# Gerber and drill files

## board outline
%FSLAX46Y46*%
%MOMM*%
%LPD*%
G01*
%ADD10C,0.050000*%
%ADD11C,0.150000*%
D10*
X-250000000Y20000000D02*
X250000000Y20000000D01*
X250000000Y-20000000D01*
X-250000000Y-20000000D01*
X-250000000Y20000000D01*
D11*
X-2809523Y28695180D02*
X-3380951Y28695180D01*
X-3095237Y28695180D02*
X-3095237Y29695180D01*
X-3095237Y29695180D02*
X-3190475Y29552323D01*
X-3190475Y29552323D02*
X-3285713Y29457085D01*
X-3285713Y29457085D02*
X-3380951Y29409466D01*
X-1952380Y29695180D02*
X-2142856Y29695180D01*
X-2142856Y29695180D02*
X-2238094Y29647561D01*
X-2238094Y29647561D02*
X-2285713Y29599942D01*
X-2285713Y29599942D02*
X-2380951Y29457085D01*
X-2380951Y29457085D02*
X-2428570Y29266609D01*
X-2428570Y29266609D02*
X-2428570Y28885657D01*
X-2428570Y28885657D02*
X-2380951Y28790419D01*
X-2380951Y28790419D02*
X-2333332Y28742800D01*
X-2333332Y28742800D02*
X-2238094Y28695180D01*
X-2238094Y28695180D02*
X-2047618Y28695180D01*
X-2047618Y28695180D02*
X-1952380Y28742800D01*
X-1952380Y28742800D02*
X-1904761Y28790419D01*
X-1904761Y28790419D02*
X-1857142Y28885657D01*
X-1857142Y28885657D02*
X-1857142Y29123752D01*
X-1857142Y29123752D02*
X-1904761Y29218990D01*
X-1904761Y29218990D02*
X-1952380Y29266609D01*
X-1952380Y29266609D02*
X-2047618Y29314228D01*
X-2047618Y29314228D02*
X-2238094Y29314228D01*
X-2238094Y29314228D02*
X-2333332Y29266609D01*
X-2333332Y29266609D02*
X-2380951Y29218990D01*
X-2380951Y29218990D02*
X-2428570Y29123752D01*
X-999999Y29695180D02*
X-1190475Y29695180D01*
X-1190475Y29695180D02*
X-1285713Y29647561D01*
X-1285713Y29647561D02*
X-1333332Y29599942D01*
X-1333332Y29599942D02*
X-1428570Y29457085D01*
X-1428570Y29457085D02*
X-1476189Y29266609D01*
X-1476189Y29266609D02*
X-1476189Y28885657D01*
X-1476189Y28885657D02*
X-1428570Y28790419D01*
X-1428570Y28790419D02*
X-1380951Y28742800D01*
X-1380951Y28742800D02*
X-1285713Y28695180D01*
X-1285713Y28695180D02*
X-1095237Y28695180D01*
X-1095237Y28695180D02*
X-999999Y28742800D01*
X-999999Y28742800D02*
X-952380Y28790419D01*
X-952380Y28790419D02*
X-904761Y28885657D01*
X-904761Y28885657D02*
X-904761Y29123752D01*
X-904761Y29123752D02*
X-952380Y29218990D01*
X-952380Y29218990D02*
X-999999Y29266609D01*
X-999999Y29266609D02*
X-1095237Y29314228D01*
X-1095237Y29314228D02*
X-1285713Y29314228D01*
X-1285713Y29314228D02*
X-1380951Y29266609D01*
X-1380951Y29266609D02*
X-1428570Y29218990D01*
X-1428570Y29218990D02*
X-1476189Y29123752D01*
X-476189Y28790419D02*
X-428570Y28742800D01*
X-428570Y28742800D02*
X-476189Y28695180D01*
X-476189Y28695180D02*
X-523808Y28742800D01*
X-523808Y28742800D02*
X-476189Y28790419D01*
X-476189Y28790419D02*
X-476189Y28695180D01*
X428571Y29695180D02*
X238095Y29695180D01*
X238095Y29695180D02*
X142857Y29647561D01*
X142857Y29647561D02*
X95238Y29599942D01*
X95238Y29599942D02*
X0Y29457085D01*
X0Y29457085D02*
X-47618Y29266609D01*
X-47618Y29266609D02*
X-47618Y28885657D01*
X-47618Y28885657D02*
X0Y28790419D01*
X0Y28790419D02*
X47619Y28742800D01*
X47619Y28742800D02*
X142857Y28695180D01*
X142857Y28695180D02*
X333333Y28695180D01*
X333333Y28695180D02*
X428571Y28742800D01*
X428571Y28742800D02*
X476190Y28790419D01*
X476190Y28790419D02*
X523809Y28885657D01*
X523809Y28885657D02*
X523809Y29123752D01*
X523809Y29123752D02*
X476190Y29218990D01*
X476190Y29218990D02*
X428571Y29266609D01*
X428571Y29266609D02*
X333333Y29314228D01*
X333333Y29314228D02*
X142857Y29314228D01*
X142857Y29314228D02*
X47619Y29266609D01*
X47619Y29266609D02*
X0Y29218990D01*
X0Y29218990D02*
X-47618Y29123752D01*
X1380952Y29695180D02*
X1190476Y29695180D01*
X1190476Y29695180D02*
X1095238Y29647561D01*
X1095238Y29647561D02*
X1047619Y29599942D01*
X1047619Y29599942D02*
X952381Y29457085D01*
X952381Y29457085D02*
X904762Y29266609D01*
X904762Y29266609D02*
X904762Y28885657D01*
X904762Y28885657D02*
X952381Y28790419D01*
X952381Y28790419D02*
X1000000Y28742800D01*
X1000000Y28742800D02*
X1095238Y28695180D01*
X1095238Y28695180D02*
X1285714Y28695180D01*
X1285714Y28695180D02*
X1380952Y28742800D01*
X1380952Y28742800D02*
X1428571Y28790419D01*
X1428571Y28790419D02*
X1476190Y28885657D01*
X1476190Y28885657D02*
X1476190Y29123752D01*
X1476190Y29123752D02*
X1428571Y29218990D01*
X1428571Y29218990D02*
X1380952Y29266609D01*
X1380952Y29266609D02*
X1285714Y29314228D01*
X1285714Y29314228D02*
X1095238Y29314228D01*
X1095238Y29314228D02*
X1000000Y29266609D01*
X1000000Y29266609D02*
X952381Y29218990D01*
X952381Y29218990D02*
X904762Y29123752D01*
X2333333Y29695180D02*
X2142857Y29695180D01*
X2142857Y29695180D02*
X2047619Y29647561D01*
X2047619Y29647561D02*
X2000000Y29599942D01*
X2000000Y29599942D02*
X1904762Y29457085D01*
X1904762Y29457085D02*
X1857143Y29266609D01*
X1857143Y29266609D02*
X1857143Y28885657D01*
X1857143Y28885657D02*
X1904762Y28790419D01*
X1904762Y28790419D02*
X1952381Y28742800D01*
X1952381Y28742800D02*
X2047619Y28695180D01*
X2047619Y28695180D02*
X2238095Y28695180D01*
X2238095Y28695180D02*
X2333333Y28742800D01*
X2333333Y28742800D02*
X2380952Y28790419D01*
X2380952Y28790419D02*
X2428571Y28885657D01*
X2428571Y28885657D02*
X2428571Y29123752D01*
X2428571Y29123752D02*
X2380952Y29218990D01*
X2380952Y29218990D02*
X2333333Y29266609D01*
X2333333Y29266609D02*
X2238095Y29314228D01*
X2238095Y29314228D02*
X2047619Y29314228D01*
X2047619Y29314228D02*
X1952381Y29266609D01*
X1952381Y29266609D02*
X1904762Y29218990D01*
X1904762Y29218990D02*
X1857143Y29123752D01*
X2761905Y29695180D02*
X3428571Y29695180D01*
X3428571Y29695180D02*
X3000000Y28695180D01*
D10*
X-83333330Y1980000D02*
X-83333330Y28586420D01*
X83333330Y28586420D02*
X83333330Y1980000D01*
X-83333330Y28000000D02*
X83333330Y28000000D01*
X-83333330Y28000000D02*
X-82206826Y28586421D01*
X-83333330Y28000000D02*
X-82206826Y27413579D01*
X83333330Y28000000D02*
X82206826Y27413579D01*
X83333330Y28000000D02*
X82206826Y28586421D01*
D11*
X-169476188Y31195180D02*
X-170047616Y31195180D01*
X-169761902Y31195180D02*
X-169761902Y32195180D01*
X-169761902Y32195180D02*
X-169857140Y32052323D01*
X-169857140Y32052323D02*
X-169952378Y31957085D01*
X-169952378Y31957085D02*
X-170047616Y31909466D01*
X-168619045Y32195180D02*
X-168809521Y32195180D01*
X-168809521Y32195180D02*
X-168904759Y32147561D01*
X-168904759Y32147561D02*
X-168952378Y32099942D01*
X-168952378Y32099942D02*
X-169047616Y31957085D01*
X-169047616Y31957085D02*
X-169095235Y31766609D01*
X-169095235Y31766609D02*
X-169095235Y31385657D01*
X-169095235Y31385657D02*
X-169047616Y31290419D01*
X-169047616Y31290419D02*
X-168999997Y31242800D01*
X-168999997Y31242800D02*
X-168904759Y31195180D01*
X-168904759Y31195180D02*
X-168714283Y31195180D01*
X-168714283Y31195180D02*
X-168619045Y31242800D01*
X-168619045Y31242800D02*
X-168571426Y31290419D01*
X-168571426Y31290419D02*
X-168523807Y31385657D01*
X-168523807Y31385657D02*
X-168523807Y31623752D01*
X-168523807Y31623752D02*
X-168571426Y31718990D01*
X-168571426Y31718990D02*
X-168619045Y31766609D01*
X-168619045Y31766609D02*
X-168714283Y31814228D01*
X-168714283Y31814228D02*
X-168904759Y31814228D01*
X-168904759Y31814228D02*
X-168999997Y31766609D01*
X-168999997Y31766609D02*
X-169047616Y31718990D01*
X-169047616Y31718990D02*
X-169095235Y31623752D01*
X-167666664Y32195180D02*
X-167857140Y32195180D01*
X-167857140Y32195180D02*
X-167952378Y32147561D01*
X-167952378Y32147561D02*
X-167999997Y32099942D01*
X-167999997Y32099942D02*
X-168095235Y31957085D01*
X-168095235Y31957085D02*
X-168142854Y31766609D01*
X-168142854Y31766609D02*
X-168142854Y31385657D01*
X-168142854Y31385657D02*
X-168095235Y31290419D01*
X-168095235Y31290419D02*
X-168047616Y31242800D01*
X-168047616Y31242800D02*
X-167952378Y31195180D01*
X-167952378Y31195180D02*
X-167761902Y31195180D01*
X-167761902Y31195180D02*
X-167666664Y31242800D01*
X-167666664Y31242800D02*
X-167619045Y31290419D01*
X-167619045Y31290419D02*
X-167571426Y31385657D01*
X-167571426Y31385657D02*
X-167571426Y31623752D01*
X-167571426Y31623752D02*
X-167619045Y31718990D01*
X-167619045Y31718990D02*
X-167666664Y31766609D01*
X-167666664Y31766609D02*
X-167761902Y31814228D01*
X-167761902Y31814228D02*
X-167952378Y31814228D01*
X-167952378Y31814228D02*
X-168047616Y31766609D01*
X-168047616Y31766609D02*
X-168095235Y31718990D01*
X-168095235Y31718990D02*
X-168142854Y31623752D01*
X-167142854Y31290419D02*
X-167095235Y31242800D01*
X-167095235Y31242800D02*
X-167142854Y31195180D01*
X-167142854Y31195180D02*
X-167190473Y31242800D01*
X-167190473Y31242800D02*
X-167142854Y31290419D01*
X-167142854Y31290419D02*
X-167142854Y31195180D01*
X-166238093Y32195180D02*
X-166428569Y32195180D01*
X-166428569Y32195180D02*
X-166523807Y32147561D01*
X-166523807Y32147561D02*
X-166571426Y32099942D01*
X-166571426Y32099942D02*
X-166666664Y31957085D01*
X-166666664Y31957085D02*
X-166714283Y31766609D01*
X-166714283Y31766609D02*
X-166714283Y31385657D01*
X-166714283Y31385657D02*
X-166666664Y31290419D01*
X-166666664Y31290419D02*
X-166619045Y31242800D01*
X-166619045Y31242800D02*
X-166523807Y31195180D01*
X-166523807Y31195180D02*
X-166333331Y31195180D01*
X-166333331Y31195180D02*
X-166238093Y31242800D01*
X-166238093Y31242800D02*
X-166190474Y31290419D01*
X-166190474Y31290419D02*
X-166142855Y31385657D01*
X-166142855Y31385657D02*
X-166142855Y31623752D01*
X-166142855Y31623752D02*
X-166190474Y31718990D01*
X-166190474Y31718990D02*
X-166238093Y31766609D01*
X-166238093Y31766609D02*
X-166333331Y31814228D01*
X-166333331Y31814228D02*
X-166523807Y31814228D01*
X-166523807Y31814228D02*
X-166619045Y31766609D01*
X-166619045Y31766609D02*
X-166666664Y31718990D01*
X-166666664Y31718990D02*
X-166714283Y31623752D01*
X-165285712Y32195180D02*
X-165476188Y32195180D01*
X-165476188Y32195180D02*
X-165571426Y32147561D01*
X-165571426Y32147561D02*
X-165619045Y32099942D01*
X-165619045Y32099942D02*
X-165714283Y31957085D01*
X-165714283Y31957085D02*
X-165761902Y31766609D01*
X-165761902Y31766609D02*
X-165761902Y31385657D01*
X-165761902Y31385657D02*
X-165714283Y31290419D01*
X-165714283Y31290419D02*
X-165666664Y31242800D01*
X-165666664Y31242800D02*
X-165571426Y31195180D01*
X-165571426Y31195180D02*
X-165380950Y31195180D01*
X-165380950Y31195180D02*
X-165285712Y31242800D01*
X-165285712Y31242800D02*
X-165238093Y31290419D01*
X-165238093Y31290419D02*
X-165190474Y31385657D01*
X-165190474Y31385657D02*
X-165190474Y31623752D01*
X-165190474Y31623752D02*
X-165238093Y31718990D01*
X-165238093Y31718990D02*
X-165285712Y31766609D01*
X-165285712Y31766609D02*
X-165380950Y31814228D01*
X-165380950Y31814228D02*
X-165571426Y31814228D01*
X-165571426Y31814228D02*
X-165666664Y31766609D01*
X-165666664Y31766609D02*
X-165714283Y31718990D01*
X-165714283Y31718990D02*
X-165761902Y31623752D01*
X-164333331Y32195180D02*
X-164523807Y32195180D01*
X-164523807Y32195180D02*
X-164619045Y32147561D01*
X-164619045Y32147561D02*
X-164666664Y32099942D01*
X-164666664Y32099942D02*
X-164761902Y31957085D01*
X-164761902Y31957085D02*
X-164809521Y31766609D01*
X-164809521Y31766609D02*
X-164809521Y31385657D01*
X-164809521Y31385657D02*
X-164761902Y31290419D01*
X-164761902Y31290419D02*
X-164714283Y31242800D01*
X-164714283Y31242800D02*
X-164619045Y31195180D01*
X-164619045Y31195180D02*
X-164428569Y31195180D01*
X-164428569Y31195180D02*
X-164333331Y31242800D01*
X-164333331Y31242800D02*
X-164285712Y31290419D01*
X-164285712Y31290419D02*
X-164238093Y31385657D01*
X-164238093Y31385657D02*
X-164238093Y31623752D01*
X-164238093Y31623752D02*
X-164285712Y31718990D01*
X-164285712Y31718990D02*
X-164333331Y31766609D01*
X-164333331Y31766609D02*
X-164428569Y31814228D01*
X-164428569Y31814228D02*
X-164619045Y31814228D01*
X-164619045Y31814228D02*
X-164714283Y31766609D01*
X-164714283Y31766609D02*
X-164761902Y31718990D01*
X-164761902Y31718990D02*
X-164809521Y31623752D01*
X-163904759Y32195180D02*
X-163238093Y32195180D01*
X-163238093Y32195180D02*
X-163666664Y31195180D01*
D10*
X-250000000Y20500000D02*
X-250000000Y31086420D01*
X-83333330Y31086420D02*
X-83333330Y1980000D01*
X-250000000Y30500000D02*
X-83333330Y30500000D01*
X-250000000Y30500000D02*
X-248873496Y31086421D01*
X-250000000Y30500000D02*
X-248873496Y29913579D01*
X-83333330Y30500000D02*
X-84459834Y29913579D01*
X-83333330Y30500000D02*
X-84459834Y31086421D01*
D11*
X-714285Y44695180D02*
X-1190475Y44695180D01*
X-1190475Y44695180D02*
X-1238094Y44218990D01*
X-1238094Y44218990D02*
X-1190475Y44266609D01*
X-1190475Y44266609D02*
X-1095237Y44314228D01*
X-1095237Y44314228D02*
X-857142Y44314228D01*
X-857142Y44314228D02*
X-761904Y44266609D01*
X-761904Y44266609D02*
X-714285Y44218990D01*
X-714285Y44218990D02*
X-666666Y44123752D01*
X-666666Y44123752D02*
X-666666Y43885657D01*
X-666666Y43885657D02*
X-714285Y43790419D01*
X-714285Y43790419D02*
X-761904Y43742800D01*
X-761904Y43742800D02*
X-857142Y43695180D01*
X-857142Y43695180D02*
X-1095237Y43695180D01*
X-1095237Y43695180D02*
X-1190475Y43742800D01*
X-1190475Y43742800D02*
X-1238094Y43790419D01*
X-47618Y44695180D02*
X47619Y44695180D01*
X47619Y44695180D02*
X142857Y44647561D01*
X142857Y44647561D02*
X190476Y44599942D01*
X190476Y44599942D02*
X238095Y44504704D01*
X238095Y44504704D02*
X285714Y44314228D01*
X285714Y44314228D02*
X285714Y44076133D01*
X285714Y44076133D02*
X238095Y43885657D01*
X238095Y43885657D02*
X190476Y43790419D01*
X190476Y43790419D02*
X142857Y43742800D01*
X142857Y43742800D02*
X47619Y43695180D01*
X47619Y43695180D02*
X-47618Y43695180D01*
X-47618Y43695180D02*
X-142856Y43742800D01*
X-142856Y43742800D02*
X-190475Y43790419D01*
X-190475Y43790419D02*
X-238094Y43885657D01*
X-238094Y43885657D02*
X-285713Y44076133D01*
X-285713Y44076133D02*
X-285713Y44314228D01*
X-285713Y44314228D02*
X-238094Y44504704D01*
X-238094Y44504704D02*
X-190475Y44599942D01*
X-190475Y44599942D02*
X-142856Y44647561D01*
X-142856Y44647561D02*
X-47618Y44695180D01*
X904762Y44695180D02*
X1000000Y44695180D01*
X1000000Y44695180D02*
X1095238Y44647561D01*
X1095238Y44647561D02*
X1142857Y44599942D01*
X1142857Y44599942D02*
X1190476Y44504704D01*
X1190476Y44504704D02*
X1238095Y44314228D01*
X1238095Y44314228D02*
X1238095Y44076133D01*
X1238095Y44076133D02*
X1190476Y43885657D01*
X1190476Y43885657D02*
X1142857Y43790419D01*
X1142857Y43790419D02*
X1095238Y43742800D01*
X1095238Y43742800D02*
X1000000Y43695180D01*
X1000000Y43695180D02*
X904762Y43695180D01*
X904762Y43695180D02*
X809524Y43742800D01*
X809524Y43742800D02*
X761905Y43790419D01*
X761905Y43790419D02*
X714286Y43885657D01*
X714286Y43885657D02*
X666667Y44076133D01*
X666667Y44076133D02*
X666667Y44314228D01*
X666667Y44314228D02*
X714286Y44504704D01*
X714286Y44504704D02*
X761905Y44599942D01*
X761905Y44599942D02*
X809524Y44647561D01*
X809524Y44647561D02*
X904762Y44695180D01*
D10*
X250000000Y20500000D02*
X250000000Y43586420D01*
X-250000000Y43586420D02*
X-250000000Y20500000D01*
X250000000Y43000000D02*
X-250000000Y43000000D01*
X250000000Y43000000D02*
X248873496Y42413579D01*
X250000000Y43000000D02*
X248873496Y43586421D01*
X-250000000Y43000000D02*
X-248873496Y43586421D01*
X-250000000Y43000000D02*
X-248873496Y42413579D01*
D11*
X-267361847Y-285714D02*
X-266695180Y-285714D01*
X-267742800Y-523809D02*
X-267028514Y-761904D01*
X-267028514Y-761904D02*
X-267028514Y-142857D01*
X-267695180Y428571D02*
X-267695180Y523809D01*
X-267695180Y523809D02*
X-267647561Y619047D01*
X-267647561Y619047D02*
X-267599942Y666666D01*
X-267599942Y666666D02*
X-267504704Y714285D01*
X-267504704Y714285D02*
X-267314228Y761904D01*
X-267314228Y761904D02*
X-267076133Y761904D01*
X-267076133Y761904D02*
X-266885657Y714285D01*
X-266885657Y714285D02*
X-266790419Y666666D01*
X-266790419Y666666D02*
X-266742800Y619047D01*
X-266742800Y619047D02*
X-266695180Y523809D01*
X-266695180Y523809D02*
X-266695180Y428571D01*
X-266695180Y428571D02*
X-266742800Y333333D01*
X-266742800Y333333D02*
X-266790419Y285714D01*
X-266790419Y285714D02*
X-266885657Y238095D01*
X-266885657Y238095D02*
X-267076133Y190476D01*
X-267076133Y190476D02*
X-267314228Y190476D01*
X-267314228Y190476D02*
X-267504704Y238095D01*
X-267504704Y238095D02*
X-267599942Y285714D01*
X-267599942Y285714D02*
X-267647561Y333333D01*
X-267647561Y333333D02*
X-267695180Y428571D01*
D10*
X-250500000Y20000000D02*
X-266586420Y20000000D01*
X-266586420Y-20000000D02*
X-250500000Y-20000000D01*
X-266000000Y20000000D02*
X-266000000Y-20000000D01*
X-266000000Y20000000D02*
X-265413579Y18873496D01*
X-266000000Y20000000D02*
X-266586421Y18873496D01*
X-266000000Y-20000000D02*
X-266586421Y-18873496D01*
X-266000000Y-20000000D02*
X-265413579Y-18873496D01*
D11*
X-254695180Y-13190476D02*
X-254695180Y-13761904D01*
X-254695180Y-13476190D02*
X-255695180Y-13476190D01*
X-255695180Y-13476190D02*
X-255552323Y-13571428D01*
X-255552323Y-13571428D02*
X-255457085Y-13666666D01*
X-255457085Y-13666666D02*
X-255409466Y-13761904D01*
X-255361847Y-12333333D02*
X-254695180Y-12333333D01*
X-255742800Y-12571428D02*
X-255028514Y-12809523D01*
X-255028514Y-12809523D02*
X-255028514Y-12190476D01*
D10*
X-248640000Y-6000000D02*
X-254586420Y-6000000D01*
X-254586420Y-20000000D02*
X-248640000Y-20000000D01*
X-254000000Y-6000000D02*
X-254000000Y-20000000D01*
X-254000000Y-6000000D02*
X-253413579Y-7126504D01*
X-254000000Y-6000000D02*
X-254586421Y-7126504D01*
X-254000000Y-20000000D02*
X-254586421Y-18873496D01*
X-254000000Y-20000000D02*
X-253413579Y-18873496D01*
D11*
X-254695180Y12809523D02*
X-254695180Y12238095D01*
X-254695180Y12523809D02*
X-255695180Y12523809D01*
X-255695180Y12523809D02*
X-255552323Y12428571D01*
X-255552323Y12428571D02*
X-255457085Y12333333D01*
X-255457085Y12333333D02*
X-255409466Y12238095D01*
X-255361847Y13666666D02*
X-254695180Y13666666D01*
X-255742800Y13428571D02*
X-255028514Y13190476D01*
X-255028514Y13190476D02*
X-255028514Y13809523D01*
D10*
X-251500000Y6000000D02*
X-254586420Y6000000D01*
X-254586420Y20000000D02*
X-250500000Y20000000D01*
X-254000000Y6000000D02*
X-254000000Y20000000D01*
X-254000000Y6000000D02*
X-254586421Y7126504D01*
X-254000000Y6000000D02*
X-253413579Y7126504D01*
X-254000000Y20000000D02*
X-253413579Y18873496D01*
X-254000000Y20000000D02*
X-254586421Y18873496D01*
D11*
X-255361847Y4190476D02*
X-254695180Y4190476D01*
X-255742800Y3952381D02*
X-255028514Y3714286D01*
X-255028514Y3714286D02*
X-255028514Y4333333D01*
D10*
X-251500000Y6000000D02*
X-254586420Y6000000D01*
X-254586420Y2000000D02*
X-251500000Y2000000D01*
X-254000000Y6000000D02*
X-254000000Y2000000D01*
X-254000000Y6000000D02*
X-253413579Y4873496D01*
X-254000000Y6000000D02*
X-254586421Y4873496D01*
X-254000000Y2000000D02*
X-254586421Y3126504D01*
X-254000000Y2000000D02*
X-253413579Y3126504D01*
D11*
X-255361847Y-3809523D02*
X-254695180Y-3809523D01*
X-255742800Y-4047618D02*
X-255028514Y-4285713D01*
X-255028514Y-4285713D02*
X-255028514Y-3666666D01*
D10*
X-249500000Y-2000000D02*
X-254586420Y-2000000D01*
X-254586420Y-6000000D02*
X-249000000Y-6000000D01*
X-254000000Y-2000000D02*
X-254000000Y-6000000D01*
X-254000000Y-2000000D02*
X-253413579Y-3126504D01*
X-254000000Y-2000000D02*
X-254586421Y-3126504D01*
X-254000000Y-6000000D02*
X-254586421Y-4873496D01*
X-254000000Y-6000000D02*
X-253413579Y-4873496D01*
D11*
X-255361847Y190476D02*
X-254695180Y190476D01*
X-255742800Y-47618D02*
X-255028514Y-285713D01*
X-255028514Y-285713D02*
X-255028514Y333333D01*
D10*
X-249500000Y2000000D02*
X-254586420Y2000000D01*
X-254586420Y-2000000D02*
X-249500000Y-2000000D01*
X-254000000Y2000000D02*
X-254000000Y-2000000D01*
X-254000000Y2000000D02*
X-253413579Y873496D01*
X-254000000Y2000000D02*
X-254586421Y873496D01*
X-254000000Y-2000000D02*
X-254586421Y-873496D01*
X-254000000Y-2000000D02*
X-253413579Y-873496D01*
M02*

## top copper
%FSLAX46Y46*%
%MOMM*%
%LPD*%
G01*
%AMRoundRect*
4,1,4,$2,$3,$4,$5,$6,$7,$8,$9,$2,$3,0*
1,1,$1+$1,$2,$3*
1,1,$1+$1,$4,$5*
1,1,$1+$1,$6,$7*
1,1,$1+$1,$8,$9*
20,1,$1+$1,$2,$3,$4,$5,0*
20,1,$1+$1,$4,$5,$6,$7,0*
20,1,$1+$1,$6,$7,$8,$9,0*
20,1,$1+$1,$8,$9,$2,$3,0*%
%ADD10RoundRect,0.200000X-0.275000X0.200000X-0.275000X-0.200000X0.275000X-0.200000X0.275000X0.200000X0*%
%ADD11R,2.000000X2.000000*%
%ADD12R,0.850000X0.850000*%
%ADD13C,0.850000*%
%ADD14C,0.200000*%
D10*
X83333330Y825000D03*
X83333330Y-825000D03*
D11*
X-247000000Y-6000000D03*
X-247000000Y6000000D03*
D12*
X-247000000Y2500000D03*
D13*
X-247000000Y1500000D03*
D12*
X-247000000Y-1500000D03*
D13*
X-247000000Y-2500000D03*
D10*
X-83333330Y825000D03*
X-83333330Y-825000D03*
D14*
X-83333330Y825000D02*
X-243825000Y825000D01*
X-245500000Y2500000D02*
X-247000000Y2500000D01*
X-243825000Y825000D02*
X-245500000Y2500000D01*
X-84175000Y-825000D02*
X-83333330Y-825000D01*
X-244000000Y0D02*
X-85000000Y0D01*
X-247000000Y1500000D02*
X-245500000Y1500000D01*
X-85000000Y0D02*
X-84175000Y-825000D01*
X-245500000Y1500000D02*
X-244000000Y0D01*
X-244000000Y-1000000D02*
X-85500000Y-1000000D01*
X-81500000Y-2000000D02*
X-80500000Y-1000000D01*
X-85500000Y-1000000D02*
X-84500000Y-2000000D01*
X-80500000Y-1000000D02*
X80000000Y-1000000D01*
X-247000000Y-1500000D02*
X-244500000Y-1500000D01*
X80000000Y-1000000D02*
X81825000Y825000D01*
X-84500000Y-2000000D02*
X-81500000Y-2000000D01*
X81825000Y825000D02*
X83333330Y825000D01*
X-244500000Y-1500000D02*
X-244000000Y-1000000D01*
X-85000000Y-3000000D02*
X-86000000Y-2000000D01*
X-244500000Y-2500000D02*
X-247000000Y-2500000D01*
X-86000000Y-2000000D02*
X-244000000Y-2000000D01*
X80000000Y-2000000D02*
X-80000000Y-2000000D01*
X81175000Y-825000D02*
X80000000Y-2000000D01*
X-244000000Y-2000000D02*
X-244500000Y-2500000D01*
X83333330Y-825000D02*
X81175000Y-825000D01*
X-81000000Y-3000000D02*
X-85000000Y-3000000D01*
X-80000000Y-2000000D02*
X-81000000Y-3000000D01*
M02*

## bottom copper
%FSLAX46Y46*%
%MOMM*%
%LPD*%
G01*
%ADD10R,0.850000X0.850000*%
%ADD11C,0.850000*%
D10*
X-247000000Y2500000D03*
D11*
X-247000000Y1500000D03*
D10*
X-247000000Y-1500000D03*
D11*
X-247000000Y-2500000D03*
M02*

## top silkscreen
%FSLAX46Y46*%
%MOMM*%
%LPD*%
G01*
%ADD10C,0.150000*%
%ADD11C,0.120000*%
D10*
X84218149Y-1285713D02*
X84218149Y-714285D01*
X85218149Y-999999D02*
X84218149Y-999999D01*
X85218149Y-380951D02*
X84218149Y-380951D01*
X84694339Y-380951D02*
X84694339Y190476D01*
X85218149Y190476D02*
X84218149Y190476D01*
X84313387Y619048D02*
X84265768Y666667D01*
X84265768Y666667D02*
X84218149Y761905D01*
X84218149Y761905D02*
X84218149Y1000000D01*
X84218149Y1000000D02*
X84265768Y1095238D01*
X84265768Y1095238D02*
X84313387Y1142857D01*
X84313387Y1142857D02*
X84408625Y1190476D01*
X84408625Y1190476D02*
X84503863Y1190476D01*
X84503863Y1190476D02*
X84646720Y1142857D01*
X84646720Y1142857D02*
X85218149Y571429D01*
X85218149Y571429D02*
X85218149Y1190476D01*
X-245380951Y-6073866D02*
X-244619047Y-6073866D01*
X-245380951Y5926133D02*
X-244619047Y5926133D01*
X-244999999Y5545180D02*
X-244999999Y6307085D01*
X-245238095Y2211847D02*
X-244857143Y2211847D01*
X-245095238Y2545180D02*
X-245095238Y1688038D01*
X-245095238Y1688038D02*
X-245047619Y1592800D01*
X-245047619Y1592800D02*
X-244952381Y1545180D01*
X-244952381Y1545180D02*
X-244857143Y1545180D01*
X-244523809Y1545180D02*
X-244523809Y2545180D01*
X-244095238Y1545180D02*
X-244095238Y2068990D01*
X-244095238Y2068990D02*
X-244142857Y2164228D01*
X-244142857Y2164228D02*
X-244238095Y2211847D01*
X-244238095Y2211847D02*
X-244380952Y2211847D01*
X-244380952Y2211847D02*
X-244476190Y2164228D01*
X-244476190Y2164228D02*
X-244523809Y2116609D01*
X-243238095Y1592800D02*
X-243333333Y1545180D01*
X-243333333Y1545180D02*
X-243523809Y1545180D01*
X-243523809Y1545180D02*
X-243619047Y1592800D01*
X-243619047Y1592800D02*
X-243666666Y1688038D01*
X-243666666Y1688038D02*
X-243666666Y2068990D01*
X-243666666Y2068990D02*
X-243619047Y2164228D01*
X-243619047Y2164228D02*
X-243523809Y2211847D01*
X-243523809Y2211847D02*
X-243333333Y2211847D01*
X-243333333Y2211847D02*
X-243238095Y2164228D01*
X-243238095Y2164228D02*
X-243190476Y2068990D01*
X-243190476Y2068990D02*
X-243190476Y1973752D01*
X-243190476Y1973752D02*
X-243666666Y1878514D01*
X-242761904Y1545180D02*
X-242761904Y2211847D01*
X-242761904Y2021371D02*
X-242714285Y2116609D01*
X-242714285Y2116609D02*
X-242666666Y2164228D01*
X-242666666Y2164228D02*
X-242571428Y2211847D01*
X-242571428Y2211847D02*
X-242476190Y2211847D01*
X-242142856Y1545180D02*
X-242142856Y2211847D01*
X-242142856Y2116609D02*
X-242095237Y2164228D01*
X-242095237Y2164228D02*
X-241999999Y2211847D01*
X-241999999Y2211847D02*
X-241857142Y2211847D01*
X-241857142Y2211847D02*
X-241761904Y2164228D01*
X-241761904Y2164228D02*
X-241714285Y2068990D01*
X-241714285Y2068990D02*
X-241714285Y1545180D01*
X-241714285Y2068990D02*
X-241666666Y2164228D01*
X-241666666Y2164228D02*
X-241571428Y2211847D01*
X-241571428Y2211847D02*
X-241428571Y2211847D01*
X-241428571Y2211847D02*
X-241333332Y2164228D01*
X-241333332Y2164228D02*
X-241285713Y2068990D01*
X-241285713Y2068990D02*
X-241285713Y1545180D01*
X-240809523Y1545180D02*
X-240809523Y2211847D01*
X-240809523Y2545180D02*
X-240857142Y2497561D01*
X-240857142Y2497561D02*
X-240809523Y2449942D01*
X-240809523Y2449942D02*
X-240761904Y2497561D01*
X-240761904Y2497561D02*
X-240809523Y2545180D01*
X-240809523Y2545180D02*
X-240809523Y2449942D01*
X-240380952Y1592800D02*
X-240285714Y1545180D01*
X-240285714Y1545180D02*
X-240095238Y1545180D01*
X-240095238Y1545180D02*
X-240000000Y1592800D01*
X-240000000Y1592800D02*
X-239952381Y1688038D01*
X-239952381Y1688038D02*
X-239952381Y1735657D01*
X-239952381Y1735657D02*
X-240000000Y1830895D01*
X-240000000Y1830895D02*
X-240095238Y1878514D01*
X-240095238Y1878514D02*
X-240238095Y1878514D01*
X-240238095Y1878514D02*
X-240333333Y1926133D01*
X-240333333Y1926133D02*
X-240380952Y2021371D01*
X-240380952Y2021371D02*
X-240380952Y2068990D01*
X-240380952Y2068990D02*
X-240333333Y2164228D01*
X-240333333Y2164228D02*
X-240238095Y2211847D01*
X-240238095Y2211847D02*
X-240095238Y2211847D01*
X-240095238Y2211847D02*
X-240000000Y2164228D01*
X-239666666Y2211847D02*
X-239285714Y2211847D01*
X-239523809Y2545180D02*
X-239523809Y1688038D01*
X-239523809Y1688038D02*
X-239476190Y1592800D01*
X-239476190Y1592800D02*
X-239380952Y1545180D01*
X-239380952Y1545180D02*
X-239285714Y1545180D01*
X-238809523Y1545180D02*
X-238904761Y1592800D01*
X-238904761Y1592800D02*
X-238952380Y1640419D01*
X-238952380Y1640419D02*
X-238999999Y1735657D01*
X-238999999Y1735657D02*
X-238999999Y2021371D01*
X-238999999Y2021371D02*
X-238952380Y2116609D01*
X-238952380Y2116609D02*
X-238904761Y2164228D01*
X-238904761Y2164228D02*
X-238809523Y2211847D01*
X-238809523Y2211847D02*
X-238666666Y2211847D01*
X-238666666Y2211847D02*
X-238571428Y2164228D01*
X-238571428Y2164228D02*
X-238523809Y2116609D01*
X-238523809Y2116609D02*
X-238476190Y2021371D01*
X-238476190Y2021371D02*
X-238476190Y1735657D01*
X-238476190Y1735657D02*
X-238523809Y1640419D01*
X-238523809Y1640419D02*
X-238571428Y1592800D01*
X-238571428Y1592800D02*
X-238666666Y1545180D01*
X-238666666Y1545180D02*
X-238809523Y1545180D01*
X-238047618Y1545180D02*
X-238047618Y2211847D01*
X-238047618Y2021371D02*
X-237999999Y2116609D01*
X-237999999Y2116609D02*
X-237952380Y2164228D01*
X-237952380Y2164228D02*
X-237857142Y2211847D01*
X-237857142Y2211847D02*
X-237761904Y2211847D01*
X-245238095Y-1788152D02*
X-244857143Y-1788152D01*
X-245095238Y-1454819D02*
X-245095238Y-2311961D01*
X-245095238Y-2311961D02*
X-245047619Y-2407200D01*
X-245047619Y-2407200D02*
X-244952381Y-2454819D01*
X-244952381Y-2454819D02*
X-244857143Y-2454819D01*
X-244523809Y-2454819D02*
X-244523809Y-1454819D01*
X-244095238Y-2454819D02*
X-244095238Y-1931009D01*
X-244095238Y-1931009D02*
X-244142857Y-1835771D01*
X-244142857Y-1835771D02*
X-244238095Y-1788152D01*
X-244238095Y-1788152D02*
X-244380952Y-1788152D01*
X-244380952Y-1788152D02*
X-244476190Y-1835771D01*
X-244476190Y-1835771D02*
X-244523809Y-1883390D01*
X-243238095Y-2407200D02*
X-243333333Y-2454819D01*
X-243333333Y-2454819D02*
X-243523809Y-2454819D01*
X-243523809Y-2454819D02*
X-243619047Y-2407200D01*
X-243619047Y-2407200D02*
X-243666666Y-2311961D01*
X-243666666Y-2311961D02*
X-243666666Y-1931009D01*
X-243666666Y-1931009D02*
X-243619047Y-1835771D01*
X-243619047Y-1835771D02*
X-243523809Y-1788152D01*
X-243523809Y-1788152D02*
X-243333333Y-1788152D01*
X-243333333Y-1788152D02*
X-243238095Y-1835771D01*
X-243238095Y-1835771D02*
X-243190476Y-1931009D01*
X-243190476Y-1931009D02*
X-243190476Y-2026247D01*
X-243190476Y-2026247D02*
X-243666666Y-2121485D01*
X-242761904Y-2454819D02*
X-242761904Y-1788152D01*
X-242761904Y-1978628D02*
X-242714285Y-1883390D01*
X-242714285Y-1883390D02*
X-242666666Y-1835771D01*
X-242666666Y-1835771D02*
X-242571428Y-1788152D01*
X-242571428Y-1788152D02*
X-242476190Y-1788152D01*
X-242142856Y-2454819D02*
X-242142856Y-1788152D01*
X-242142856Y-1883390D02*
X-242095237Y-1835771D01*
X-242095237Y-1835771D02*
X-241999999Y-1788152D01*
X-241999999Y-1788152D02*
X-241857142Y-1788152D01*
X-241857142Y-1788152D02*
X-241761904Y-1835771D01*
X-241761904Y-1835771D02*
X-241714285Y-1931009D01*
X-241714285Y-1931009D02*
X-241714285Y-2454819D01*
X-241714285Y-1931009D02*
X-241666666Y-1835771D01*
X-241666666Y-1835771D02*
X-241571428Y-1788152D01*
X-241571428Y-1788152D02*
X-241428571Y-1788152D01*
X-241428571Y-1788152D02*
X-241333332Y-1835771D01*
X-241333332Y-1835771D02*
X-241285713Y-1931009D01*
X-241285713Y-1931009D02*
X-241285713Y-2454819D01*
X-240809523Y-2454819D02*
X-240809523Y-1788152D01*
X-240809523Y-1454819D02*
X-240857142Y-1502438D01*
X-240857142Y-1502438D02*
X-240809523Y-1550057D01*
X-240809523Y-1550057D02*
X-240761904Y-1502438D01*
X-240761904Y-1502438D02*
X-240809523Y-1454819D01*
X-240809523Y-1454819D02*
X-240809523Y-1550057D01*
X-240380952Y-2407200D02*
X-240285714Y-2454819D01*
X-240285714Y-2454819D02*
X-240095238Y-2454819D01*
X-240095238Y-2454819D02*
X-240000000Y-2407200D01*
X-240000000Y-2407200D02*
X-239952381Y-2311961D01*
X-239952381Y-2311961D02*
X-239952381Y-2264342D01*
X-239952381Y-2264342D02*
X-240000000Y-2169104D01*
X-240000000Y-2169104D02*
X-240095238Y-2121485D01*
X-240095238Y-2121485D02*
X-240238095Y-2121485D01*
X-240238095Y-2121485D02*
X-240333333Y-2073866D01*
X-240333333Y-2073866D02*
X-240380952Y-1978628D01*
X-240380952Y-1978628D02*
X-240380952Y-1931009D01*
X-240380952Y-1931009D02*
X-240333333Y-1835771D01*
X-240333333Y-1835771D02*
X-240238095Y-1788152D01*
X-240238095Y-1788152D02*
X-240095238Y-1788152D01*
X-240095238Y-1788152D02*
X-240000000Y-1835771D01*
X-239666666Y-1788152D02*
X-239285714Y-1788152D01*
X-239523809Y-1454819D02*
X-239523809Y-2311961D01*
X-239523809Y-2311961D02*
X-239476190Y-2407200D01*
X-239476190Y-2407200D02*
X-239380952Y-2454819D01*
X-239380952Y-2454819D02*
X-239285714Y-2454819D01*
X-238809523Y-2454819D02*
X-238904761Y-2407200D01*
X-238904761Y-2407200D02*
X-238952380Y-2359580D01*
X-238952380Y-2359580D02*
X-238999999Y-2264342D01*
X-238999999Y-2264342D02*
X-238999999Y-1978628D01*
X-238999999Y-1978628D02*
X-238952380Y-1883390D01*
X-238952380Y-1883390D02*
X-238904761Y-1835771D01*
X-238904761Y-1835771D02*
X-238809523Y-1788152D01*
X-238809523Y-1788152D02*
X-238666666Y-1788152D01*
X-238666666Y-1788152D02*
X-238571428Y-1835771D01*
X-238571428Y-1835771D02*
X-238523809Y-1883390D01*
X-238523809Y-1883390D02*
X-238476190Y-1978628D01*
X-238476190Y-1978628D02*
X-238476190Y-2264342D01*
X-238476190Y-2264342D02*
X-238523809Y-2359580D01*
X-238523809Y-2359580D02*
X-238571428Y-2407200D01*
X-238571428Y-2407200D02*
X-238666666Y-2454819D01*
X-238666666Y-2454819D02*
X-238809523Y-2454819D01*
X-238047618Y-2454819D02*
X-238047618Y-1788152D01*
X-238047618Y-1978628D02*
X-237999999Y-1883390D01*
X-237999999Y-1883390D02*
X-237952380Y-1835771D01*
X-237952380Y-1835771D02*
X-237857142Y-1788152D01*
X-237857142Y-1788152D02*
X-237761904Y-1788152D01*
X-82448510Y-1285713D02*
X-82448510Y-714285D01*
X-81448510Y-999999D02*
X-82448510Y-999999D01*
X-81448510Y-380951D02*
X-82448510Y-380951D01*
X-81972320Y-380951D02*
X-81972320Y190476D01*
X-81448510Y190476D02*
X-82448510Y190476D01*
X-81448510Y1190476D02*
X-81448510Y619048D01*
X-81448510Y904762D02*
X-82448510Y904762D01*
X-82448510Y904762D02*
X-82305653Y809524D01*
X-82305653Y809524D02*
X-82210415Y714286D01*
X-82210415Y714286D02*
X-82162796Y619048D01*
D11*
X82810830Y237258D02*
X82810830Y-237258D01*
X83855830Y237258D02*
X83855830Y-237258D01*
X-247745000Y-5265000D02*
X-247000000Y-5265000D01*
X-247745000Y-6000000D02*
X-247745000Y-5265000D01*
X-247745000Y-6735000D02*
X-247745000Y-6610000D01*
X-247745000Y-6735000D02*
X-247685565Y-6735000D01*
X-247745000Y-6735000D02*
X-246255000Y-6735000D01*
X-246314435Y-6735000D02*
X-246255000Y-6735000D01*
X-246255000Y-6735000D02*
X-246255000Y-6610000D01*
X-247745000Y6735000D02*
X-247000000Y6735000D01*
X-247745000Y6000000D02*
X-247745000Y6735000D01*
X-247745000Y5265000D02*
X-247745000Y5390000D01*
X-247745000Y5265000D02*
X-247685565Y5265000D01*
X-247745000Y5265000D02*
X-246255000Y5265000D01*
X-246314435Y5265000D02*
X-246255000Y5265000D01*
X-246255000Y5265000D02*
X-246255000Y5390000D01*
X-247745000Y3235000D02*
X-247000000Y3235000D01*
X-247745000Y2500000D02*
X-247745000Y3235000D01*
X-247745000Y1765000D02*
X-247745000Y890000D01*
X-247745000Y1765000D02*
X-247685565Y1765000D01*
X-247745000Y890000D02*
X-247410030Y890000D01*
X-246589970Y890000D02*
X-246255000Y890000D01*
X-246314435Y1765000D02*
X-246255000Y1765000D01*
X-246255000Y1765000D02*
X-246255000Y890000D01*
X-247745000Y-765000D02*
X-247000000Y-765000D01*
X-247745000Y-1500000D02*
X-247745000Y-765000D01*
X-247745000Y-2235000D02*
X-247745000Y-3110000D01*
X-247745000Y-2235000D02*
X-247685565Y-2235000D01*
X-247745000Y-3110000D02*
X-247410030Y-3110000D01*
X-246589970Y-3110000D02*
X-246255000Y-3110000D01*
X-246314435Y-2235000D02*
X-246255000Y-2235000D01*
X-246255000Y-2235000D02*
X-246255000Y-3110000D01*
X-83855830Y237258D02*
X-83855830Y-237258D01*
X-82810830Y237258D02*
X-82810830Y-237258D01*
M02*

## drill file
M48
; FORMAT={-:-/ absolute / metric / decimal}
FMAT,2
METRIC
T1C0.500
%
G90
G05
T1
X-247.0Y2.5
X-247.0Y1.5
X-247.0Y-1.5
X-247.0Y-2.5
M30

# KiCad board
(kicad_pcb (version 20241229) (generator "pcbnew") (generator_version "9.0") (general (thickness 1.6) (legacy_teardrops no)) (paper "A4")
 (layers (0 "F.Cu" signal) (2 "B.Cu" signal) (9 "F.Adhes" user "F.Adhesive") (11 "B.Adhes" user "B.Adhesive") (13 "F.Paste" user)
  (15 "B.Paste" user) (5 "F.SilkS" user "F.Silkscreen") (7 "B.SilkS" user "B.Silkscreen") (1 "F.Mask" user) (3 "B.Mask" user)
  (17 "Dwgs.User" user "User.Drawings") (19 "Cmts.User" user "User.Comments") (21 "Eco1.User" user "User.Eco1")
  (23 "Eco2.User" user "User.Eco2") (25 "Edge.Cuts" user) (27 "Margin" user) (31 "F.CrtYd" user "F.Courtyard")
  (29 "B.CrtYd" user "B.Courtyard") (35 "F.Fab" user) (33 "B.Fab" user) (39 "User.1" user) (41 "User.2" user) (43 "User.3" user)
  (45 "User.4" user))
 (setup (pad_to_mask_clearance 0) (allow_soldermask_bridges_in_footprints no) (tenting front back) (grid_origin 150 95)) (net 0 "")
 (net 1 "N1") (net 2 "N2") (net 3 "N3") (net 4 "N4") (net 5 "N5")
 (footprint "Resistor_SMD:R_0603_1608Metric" (layer "F.Cu") (at 83.33333 0 -90)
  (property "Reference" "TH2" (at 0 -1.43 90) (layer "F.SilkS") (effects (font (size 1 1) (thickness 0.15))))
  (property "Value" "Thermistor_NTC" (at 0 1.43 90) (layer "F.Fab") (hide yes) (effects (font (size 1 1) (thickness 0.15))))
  (fp_line (start -0.237258 0.5225) (end 0.237258 0.5225) (stroke (width 0.12) (type solid)) (layer "F.SilkS"))
  (fp_line (start -0.237258 -0.5225) (end 0.237258 -0.5225) (stroke (width 0.12) (type solid)) (layer "F.SilkS"))
  (pad "1" smd roundrect (at -0.825 0 270) (size 0.8 0.95) (layers "F.Cu" "F.Mask" "F.Paste") (roundrect_rratio 0.25) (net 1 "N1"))
  (pad "2" smd roundrect (at 0.825 0 270) (size 0.8 0.95) (layers "F.Cu" "F.Mask" "F.Paste") (roundrect_rratio 0.25) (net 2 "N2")))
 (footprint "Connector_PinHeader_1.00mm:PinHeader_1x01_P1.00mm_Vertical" (layer "F.Cu") (at -247 6)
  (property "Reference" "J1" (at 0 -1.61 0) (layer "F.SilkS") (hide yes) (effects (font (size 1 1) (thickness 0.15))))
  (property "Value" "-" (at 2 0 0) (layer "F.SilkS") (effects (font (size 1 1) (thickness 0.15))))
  (fp_line (start -0.745 -0.735) (end 0 -0.735) (stroke (width 0.12) (type solid)) (layer "F.SilkS"))
  (fp_line (start -0.745 0) (end -0.745 -0.735) (stroke (width 0.12) (type solid)) (layer "F.SilkS"))
  (fp_line (start -0.745 0.735) (end -0.745 0.61) (stroke (width 0.12) (type solid)) (layer "F.SilkS"))
  (fp_line (start -0.745 0.735) (end -0.685565 0.735) (stroke (width 0.12) (type solid)) (layer "F.SilkS"))
  (fp_line (start -0.745 0.735) (end 0.745 0.735) (stroke (width 0.12) (type solid)) (layer "F.SilkS"))
  (fp_line (start 0.685565 0.735) (end 0.745 0.735) (stroke (width 0.12) (type solid)) (layer "F.SilkS"))
  (fp_line (start 0.745 0.735) (end 0.745 0.61) (stroke (width 0.12) (type solid)) (layer "F.SilkS"))
  (pad "1" smd rect (at 0 0) (size 2 2) (layers "F.Cu" "F.Mask" "F.Paste") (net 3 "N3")))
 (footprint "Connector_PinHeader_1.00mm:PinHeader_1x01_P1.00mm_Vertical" (layer "F.Cu") (at -247 -6)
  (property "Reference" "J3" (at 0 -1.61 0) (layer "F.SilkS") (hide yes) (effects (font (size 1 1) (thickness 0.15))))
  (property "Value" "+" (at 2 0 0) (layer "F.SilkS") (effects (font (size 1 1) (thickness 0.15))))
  (fp_line (start -0.745 -0.735) (end 0 -0.735) (stroke (width 0.12) (type solid)) (layer "F.SilkS"))
  (fp_line (start -0.745 0) (end -0.745 -0.735) (stroke (width 0.12) (type solid)) (layer "F.SilkS"))
  (fp_line (start -0.745 0.735) (end -0.745 0.61) (stroke (width 0.12) (type solid)) (layer "F.SilkS"))
  (fp_line (start -0.745 0.735) (end -0.685565 0.735) (stroke (width 0.12) (type solid)) (layer "F.SilkS"))
  (fp_line (start -0.745 0.735) (end 0.745 0.735) (stroke (width 0.12) (type solid)) (layer "F.SilkS"))
  (fp_line (start 0.685565 0.735) (end 0.745 0.735) (stroke (width 0.12) (type solid)) (layer "F.SilkS"))
  (fp_line (start 0.745 0.735) (end 0.745 0.61) (stroke (width 0.12) (type solid)) (layer "F.SilkS"))
  (pad "1" smd rect (at 0 0) (size 2 2) (layers "F.Cu" "F.Mask" "F.Paste") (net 3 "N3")))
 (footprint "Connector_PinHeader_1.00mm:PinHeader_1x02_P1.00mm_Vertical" (layer "F.Cu") (at -247 -2.5)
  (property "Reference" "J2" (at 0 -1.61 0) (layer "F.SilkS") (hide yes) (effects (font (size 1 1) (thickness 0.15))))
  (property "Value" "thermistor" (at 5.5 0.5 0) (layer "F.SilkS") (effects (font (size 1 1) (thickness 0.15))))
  (fp_line (start -0.745 -0.735) (end 0 -0.735) (stroke (width 0.12) (type solid)) (layer "F.SilkS"))
  (fp_line (start -0.745 0) (end -0.745 -0.735) (stroke (width 0.12) (type solid)) (layer "F.SilkS"))
  (fp_line (start -0.745 0.735) (end -0.745 1.61) (stroke (width 0.12) (type solid)) (layer "F.SilkS"))
  (fp_line (start -0.745 0.735) (end -0.685565 0.735) (stroke (width 0.12) (type solid)) (layer "F.SilkS"))
  (fp_line (start -0.745 1.61) (end -0.41003 1.61) (stroke (width 0.12) (type solid)) (layer "F.SilkS"))
  (fp_line (start 0.41003 1.61) (end 0.745 1.61) (stroke (width 0.12) (type solid)) (layer "F.SilkS"))
  (fp_line (start 0.685565 0.735) (end 0.745 0.735) (stroke (width 0.12) (type solid)) (layer "F.SilkS"))
  (fp_line (start 0.745 0.735) (end 0.745 1.61) (stroke (width 0.12) (type solid)) (layer "F.SilkS"))
  (pad "1" thru_hole rect (at 0 0) (size 0.85 0.85) (drill 0.5) (layers "*.Cu" "*.Mask") (remove_unused_layers no) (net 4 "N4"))
  (pad "2" thru_hole circle (at 0 1) (size 0.85 0.85) (drill 0.5) (layers "*.Cu" "*.Mask") (remove_unused_layers no) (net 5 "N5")))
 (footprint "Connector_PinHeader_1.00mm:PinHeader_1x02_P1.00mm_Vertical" (layer "F.Cu") (at -247 1.5)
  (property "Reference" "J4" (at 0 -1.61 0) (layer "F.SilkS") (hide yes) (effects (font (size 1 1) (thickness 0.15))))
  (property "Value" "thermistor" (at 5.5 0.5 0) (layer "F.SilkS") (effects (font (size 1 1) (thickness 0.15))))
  (fp_line (start -0.745 -0.735) (end 0 -0.735) (stroke (width 0.12) (type solid)) (layer "F.SilkS"))
  (fp_line (start -0.745 0) (end -0.745 -0.735) (stroke (width 0.12) (type solid)) (layer "F.SilkS"))
  (fp_line (start -0.745 0.735) (end -0.745 1.61) (stroke (width 0.12) (type solid)) (layer "F.SilkS"))
  (fp_line (start -0.745 0.735) (end -0.685565 0.735) (stroke (width 0.12) (type solid)) (layer "F.SilkS"))
  (fp_line (start -0.745 1.61) (end -0.41003 1.61) (stroke (width 0.12) (type solid)) (layer "F.SilkS"))
  (fp_line (start 0.41003 1.61) (end 0.745 1.61) (stroke (width 0.12) (type solid)) (layer "F.SilkS"))
  (fp_line (start 0.685565 0.735) (end 0.745 0.735) (stroke (width 0.12) (type solid)) (layer "F.SilkS"))
  (fp_line (start 0.745 0.735) (end 0.745 1.61) (stroke (width 0.12) (type solid)) (layer "F.SilkS"))
  (pad "1" thru_hole rect (at 0 0) (size 0.85 0.85) (drill 0.5) (layers "*.Cu" "*.Mask") (remove_unused_layers no) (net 1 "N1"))
  (pad "2" thru_hole circle (at 0 1) (size 0.85 0.85) (drill 0.5) (layers "*.Cu" "*.Mask") (remove_unused_layers no) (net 2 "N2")))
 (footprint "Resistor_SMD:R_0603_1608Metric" (layer "F.Cu") (at -83.33333 0 -90)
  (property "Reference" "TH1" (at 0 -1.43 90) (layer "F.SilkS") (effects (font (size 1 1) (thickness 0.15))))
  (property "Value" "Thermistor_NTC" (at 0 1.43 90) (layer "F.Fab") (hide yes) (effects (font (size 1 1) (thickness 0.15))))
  (fp_line (start -0.237258 0.5225) (end 0.237258 0.5225) (stroke (width 0.12) (type solid)) (layer "F.SilkS"))
  (fp_line (start -0.237258 -0.5225) (end 0.237258 -0.5225) (stroke (width 0.12) (type solid)) (layer "F.SilkS"))
  (pad "1" smd roundrect (at -0.825 0 270) (size 0.8 0.95) (layers "F.Cu" "F.Mask" "F.Paste") (roundrect_rratio 0.25) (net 4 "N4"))
  (pad "2" smd roundrect (at 0.825 0 270) (size 0.8 0.95) (layers "F.Cu" "F.Mask" "F.Paste") (roundrect_rratio 0.25) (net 5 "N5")))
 (gr_rect (start -250 -20) (end 250 20) (stroke (width 0.05) (type solid)) (fill no) (layer "Edge.Cuts"))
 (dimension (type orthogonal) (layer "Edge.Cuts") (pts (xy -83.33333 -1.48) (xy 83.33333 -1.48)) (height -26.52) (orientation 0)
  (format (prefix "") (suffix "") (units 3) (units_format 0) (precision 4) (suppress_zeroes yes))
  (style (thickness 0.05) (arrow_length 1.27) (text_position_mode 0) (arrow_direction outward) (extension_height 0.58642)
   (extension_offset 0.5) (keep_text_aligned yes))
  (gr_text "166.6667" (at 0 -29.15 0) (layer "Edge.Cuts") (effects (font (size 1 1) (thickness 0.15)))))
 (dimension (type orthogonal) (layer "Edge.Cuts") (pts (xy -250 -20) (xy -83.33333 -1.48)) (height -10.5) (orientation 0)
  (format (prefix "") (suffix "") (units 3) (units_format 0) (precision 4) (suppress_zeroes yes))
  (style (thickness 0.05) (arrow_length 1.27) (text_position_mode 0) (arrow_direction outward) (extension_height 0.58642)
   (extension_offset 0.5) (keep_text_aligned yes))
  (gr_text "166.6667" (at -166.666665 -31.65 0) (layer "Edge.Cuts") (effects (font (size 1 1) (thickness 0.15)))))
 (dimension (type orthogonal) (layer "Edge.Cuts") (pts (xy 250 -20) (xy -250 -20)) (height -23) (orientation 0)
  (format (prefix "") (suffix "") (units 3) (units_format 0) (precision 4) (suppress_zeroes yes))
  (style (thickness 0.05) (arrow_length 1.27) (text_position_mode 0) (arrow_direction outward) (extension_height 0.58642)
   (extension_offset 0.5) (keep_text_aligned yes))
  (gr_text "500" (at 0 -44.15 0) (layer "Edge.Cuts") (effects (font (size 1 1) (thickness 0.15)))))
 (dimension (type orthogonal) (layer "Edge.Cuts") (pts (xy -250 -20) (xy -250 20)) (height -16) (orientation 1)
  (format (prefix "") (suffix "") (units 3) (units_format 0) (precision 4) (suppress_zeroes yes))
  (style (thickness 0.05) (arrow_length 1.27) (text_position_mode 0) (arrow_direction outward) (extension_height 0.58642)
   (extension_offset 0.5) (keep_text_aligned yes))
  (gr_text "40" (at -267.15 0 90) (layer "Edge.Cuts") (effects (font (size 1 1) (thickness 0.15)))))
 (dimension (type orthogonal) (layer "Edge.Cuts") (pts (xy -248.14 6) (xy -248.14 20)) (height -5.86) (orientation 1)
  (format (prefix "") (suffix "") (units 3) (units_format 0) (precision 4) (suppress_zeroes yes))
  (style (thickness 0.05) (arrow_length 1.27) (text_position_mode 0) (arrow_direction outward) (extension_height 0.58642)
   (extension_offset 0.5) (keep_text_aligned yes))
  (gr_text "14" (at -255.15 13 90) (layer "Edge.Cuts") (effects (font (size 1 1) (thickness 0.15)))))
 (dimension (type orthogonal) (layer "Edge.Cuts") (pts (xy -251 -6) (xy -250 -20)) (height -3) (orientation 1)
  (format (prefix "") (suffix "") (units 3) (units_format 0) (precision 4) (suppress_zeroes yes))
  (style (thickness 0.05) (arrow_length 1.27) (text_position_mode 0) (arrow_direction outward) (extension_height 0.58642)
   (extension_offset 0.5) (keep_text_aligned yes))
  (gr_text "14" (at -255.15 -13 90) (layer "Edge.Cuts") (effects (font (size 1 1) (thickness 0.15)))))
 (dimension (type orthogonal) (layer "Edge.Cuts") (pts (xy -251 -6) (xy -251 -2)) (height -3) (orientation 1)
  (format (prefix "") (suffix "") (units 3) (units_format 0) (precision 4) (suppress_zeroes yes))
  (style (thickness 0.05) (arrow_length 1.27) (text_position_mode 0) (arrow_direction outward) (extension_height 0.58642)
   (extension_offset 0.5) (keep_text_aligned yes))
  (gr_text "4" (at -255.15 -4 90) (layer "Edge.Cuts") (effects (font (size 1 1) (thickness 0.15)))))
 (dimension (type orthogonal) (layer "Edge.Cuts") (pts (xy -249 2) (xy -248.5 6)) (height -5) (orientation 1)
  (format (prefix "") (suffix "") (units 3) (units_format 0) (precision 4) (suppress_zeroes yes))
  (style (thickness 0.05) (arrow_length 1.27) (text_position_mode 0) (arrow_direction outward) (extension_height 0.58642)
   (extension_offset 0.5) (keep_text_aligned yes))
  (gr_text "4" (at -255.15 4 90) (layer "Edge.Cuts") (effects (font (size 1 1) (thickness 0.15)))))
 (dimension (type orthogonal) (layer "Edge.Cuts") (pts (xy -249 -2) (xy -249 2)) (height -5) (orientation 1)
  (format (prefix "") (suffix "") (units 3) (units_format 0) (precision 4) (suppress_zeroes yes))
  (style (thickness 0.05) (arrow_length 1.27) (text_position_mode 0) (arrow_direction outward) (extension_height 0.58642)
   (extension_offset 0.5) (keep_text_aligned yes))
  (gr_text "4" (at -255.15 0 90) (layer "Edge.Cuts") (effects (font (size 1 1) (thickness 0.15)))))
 (segment (start -83.33333 -0.825) (end -243.825 -0.825) (width 0.2) (layer "F.Cu") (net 4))
 (segment (start -245.5 -2.5) (end -247 -2.5) (width 0.2) (layer "F.Cu") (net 4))
 (segment (start -243.825 -0.825) (end -245.5 -2.5) (width 0.2) (layer "F.Cu") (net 4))
 (segment (start -84.175 0.825) (end -83.33333 0.825) (width 0.2) (layer "F.Cu") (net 5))
 (segment (start -244 0) (end -85 0) (width 0.2) (layer "F.Cu") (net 5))
 (segment (start -247 -1.5) (end -245.5 -1.5) (width 0.2) (layer "F.Cu") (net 5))
 (segment (start -85 0) (end -84.175 0.825) (width 0.2) (layer "F.Cu") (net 5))
 (segment (start -245.5 -1.5) (end -244 0) (width 0.2) (layer "F.Cu") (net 5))
 (segment (start -244 1) (end -85.5 1) (width 0.2) (layer "F.Cu") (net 1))
 (segment (start -81.5 2) (end -80.5 1) (width 0.2) (layer "F.Cu") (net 1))
 (segment (start -85.5 1) (end -84.5 2) (width 0.2) (layer "F.Cu") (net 1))
 (segment (start -80.5 1) (end 80 1) (width 0.2) (layer "F.Cu") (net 1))
 (segment (start -247 1.5) (end -244.5 1.5) (width 0.2) (layer "F.Cu") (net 1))
 (segment (start 80 1) (end 81.825 -0.825) (width 0.2) (layer "F.Cu") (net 1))
 (segment (start -84.5 2) (end -81.5 2) (width 0.2) (layer "F.Cu") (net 1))
 (segment (start 81.825 -0.825) (end 83.33333 -0.825) (width 0.2) (layer "F.Cu") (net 1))
 (segment (start -244.5 1.5) (end -244 1) (width 0.2) (layer "F.Cu") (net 1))
 (segment (start -85 3) (end -86 2) (width 0.2) (layer "F.Cu") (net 2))
 (segment (start -244.5 2.5) (end -247 2.5) (width 0.2) (layer "F.Cu") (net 2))
 (segment (start -86 2) (end -244 2) (width 0.2) (layer "F.Cu") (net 2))
 (segment (start 80 2) (end -80 2) (width 0.2) (layer "F.Cu") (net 2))
 (segment (start 81.175 0.825) (end 80 2) (width 0.2) (layer "F.Cu") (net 2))
 (segment (start -244 2) (end -244.5 2.5) (width 0.2) (layer "F.Cu") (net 2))
 (segment (start 83.33333 0.825) (end 81.175 0.825) (width 0.2) (layer "F.Cu") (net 2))
 (segment (start -81 3) (end -85 3) (width 0.2) (layer "F.Cu") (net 2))
 (segment (start -80 2) (end -81 3) (width 0.2) (layer "F.Cu") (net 2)))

